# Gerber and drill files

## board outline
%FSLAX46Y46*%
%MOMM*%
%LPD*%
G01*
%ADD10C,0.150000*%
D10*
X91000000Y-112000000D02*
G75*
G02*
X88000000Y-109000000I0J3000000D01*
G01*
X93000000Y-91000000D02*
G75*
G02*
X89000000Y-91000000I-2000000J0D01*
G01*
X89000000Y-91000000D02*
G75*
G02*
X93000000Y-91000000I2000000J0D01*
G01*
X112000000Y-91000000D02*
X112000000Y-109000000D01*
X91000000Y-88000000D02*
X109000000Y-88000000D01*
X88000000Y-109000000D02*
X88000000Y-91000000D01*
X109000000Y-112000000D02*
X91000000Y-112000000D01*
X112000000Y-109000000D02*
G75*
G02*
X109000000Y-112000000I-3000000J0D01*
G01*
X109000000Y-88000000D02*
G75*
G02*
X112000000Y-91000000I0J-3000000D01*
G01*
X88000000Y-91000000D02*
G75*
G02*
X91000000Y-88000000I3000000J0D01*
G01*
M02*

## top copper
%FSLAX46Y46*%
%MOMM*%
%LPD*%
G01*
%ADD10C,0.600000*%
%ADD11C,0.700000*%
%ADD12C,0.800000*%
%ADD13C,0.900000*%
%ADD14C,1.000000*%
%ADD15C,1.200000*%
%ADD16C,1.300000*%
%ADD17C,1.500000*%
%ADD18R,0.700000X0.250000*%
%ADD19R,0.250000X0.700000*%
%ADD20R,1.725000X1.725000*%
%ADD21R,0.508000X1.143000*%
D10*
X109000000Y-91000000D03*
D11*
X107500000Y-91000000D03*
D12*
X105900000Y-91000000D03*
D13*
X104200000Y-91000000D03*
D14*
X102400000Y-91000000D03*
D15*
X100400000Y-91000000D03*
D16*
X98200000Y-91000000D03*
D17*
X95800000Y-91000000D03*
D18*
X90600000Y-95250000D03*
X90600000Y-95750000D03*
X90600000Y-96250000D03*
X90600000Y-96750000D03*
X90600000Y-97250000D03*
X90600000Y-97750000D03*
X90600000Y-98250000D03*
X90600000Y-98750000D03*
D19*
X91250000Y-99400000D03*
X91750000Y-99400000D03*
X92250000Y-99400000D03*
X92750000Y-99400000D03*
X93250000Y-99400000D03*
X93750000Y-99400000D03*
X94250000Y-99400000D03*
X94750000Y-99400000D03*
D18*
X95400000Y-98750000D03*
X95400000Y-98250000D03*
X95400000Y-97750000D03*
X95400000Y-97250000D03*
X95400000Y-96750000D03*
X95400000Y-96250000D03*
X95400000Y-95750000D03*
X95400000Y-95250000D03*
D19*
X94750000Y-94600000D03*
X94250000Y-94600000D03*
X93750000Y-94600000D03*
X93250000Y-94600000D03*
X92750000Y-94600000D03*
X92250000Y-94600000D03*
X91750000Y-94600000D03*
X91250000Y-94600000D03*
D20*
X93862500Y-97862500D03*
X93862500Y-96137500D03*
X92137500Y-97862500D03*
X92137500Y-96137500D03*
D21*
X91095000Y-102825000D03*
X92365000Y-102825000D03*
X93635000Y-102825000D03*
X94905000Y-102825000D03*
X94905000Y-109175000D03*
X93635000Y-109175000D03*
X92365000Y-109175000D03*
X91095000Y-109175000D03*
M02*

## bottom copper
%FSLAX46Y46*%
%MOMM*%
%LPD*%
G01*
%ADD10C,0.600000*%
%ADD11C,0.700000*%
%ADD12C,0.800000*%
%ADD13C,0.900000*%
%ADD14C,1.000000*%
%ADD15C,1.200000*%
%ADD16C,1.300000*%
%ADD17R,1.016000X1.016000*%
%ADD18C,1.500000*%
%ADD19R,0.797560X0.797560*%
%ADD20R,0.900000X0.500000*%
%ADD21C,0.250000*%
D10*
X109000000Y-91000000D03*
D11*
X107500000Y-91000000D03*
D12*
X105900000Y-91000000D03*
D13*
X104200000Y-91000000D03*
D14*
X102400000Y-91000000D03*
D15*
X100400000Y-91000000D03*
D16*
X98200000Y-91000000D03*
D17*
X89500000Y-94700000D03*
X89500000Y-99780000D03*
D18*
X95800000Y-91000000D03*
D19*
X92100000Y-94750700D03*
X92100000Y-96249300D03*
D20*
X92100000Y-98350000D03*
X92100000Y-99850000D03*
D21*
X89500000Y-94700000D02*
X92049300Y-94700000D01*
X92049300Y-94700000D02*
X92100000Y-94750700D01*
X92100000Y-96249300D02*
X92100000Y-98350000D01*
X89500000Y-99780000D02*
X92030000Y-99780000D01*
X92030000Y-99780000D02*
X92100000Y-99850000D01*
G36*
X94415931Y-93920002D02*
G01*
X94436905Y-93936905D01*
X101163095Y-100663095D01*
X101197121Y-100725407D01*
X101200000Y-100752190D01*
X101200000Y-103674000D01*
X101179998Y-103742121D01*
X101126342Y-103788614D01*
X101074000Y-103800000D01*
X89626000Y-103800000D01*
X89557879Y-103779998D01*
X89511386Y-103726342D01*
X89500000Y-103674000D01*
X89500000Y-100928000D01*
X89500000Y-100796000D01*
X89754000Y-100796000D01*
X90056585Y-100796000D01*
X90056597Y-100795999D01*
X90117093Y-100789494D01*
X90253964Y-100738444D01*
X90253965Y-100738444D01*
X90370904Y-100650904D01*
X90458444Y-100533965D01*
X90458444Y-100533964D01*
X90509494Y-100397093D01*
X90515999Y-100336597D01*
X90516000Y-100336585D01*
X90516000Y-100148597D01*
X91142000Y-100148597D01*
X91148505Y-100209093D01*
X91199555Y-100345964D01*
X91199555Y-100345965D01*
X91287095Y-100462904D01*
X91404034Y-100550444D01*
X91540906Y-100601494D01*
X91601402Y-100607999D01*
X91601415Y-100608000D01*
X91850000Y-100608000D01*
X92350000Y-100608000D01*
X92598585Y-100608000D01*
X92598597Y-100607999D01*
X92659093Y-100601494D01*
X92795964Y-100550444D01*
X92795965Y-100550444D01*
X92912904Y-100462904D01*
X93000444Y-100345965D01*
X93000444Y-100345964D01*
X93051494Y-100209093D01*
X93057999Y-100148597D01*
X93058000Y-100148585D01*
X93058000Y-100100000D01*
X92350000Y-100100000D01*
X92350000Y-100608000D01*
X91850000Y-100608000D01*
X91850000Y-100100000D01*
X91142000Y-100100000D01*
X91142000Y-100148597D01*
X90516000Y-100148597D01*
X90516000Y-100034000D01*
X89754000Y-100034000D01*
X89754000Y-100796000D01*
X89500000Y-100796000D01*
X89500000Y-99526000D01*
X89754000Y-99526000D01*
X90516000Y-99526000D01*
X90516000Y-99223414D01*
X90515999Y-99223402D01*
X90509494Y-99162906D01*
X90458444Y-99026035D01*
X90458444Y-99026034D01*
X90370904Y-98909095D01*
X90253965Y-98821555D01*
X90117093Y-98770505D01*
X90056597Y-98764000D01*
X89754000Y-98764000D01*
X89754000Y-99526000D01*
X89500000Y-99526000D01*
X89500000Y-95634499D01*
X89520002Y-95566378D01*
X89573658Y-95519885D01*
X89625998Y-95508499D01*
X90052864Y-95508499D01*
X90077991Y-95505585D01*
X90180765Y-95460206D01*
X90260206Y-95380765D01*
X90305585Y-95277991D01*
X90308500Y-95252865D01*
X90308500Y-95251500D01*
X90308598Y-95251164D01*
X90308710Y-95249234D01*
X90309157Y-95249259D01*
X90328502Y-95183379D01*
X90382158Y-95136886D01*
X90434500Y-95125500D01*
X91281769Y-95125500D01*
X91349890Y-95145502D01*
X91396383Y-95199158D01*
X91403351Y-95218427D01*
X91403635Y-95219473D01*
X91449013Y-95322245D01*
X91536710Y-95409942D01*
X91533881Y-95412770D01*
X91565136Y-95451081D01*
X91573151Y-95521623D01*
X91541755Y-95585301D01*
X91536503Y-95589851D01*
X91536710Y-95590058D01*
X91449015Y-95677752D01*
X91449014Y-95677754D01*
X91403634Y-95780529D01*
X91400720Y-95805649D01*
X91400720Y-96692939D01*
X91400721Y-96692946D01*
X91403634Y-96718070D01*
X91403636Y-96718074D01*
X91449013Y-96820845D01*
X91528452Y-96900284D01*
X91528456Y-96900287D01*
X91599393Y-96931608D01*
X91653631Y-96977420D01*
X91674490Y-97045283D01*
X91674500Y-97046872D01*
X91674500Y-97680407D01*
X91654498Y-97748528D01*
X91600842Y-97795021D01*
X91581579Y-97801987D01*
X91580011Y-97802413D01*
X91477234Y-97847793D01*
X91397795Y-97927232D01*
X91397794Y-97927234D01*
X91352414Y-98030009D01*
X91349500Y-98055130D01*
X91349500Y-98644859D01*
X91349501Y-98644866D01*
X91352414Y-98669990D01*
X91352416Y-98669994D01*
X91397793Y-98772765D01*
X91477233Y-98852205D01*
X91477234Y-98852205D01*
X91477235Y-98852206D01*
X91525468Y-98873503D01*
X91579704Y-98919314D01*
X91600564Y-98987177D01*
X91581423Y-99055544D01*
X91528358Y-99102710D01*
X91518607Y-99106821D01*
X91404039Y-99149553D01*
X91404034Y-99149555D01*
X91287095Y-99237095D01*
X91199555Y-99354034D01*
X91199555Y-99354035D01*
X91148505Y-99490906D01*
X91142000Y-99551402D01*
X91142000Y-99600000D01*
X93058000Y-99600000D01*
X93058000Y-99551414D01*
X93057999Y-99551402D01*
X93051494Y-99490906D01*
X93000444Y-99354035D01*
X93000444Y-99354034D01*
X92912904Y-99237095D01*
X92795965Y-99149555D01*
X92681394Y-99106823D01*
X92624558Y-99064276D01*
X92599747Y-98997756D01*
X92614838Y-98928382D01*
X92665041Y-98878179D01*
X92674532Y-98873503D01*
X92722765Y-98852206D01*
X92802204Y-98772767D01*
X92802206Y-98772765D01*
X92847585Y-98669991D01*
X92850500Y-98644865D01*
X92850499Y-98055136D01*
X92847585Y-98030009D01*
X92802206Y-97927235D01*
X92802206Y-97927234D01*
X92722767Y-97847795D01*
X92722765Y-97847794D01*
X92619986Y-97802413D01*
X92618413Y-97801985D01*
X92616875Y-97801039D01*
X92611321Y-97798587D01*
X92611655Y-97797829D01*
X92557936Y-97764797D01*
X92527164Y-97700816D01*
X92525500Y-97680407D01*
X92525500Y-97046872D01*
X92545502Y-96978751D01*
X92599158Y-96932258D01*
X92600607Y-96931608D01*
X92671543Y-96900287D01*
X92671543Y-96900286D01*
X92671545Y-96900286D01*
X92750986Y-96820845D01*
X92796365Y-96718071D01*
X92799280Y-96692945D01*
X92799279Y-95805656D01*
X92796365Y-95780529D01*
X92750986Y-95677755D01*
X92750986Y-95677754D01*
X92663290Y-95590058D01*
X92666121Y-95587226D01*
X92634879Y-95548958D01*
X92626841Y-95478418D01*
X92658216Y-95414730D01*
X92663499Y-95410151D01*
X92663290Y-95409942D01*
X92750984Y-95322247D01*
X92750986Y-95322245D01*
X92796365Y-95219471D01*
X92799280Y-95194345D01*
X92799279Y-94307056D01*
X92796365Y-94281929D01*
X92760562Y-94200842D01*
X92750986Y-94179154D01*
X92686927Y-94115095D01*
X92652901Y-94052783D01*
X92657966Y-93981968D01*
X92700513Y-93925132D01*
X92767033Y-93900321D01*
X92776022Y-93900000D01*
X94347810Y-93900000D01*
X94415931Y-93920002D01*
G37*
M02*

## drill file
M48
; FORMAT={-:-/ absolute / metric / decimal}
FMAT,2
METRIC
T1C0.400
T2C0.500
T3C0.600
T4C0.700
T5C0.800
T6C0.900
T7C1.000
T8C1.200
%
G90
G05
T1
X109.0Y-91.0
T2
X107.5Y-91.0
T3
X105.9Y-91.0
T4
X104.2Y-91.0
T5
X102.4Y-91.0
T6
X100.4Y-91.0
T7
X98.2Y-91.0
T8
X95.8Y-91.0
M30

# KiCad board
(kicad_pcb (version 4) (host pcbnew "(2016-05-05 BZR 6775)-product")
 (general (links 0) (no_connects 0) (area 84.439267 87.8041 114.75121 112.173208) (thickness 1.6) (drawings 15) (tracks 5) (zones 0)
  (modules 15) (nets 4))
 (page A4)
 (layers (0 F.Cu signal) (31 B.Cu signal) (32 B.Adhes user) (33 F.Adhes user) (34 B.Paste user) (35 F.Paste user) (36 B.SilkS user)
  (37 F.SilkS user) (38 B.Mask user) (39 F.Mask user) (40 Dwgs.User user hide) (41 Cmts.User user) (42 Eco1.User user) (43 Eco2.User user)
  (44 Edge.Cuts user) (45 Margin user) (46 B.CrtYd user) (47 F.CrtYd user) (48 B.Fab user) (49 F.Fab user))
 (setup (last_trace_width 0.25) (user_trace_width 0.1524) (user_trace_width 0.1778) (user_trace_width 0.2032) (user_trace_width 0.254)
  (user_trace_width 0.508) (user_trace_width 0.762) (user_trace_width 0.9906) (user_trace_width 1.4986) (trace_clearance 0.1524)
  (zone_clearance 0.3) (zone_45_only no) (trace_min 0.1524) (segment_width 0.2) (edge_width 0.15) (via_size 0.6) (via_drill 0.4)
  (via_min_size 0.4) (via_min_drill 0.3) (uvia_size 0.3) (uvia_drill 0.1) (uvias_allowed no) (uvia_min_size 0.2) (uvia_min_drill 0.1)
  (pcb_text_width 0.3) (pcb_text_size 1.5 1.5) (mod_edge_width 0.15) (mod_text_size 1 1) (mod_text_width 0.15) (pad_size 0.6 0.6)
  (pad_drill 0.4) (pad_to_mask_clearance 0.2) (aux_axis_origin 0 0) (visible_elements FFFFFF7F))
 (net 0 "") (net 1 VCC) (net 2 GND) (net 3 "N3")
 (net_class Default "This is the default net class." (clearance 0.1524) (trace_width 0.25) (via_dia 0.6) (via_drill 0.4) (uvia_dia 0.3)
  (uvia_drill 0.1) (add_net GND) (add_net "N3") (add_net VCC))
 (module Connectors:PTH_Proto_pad (layer F.Cu) (at 109 91)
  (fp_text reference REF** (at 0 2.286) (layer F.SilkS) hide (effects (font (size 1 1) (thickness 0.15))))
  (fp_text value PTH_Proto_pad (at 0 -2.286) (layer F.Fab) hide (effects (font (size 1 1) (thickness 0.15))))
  (pad 1 thru_hole circle (at 0 0) (size 0.6 0.6) (drill 0.4) (layers *.Cu *.Mask F.SilkS)))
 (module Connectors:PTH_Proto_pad (layer F.Cu) (at 107.5 91)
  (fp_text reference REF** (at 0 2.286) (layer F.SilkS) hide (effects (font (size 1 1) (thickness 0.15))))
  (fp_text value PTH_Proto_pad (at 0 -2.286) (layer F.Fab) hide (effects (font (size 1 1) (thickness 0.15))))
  (pad 1 thru_hole circle (at 0 0) (size 0.7 0.7) (drill 0.5) (layers *.Cu *.Mask F.SilkS)))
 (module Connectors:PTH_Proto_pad (layer F.Cu) (at 105.9 91)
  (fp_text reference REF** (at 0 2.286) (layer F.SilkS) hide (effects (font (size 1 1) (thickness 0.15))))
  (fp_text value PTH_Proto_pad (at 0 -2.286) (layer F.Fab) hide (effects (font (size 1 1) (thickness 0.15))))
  (pad 1 thru_hole circle (at 0 0) (size 0.8 0.8) (drill 0.6) (layers *.Cu *.Mask F.SilkS)))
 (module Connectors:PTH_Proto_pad (layer F.Cu) (at 104.2 91)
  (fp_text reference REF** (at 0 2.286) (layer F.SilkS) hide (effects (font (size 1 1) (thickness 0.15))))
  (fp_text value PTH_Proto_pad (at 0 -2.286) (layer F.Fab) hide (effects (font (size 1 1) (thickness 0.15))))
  (pad 1 thru_hole circle (at 0 0) (size 0.9 0.9) (drill 0.7) (layers *.Cu *.Mask F.SilkS)))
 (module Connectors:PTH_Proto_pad (layer F.Cu) (at 102.4 91)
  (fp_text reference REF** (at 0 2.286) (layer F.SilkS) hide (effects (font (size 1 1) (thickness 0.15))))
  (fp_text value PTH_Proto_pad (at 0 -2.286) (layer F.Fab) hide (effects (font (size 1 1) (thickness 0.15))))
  (pad 1 thru_hole circle (at 0 0) (size 1 1) (drill 0.8) (layers *.Cu *.Mask F.SilkS)))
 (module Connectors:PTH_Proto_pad (layer F.Cu) (at 100.4 91)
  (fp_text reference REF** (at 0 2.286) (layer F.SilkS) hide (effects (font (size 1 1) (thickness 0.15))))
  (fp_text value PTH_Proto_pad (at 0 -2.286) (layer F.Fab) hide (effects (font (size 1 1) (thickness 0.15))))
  (pad 1 thru_hole circle (at 0 0) (size 1.2 1.2) (drill 0.9) (layers *.Cu *.Mask F.SilkS)))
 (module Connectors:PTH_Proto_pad (layer F.Cu) (at 98.2 91)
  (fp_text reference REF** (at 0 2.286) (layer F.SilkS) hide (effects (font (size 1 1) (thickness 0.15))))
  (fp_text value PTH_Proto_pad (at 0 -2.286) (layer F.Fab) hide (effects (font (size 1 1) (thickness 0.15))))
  (pad 1 thru_hole circle (at 0 0) (size 1.3 1.3) (drill 1) (layers *.Cu *.Mask F.SilkS)))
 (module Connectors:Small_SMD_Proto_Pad (layer B.Cu) (at 89.5 94.7)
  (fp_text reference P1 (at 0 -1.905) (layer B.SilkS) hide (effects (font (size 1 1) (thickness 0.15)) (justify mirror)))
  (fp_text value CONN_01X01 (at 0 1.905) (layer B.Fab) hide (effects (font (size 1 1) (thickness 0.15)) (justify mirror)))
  (pad 1 smd rect (at 0 0) (size 1.016 1.016) (layers B.Cu B.Paste B.Mask) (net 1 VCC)))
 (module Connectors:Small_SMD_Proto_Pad (layer B.Cu) (at 89.5 99.78)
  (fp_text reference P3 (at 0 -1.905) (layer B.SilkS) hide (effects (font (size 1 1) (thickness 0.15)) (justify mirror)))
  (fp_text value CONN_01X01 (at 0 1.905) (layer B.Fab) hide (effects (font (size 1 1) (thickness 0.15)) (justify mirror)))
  (pad 1 smd rect (at 0 0) (size 1.016 1.016) (layers B.Cu B.Paste B.Mask) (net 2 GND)))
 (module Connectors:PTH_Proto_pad (layer F.Cu) (at 95.8 91)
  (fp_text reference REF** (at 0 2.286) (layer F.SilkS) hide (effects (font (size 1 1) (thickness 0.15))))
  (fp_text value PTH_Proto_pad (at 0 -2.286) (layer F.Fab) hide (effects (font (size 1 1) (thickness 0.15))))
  (pad 1 thru_hole circle (at 0 0) (size 1.5 1.5) (drill 1.2) (layers *.Cu *.Mask F.SilkS)))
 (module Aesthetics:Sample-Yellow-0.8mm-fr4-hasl (layer B.Cu) (at 100 102.6 180)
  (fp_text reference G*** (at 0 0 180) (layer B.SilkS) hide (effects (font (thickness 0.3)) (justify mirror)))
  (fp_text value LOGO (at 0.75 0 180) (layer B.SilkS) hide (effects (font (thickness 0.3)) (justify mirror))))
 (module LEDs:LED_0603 (layer B.Cu) (at 92.1 95.5 90)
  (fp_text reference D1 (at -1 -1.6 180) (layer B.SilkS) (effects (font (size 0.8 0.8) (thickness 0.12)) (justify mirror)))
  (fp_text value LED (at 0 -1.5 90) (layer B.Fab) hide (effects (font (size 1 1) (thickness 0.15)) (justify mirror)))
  (pad 2 smd rect (at 0.7493 0 270) (size 0.79756 0.79756) (layers B.Cu B.Paste B.Mask) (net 1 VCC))
  (pad 1 smd rect (at -0.7493 0 270) (size 0.79756 0.79756) (layers B.Cu B.Paste B.Mask) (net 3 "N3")))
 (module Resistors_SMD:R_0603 (layer B.Cu) (at 92.1 99.1 270)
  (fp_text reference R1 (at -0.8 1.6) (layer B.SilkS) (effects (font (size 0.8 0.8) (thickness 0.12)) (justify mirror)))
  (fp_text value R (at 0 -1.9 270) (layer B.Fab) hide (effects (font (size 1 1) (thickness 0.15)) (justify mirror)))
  (pad 1 smd rect (at -0.75 0 270) (size 0.5 0.9) (layers B.Cu B.Paste B.Mask) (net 3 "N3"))
  (pad 2 smd rect (at 0.75 0 270) (size 0.5 0.9) (layers B.Cu B.Paste B.Mask) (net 2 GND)))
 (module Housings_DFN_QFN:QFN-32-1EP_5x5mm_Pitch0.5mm (layer F.Cu) (at 93 97)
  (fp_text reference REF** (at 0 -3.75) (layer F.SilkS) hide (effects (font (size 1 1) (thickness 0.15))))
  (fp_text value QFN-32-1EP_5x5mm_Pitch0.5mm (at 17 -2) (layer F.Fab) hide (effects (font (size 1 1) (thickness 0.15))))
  (pad 1 smd rect (at -2.4 -1.75) (size 0.7 0.25) (layers F.Cu F.Paste F.Mask))
  (pad 2 smd rect (at -2.4 -1.25) (size 0.7 0.25) (layers F.Cu F.Paste F.Mask))
  (pad 3 smd rect (at -2.4 -0.75) (size 0.7 0.25) (layers F.Cu F.Paste F.Mask))
  (pad 4 smd rect (at -2.4 -0.25) (size 0.7 0.25) (layers F.Cu F.Paste F.Mask))
  (pad 5 smd rect (at -2.4 0.25) (size 0.7 0.25) (layers F.Cu F.Paste F.Mask))
  (pad 6 smd rect (at -2.4 0.75) (size 0.7 0.25) (layers F.Cu F.Paste F.Mask))
  (pad 7 smd rect (at -2.4 1.25) (size 0.7 0.25) (layers F.Cu F.Paste F.Mask))
  (pad 8 smd rect (at -2.4 1.75) (size 0.7 0.25) (layers F.Cu F.Paste F.Mask))
  (pad 9 smd rect (at -1.75 2.4 90) (size 0.7 0.25) (layers F.Cu F.Paste F.Mask))
  (pad 10 smd rect (at -1.25 2.4 90) (size 0.7 0.25) (layers F.Cu F.Paste F.Mask))
  (pad 11 smd rect (at -0.75 2.4 90) (size 0.7 0.25) (layers F.Cu F.Paste F.Mask))
  (pad 12 smd rect (at -0.25 2.4 90) (size 0.7 0.25) (layers F.Cu F.Paste F.Mask))
  (pad 13 smd rect (at 0.25 2.4 90) (size 0.7 0.25) (layers F.Cu F.Paste F.Mask))
  (pad 14 smd rect (at 0.75 2.4 90) (size 0.7 0.25) (layers F.Cu F.Paste F.Mask))
  (pad 15 smd rect (at 1.25 2.4 90) (size 0.7 0.25) (layers F.Cu F.Paste F.Mask))
  (pad 16 smd rect (at 1.75 2.4 90) (size 0.7 0.25) (layers F.Cu F.Paste F.Mask))
  (pad 17 smd rect (at 2.4 1.75) (size 0.7 0.25) (layers F.Cu F.Paste F.Mask))
  (pad 18 smd rect (at 2.4 1.25) (size 0.7 0.25) (layers F.Cu F.Paste F.Mask))
  (pad 19 smd rect (at 2.4 0.75) (size 0.7 0.25) (layers F.Cu F.Paste F.Mask))
  (pad 20 smd rect (at 2.4 0.25) (size 0.7 0.25) (layers F.Cu F.Paste F.Mask))
  (pad 21 smd rect (at 2.4 -0.25) (size 0.7 0.25) (layers F.Cu F.Paste F.Mask))
  (pad 22 smd rect (at 2.4 -0.75) (size 0.7 0.25) (layers F.Cu F.Paste F.Mask))
  (pad 23 smd rect (at 2.4 -1.25) (size 0.7 0.25) (layers F.Cu F.Paste F.Mask))
  (pad 24 smd rect (at 2.4 -1.75) (size 0.7 0.25) (layers F.Cu F.Paste F.Mask))
  (pad 25 smd rect (at 1.75 -2.4 90) (size 0.7 0.25) (layers F.Cu F.Paste F.Mask))
  (pad 26 smd rect (at 1.25 -2.4 90) (size 0.7 0.25) (layers F.Cu F.Paste F.Mask))
  (pad 27 smd rect (at 0.75 -2.4 90) (size 0.7 0.25) (layers F.Cu F.Paste F.Mask))
  (pad 28 smd rect (at 0.25 -2.4 90) (size 0.7 0.25) (layers F.Cu F.Paste F.Mask))
  (pad 29 smd rect (at -0.25 -2.4 90) (size 0.7 0.25) (layers F.Cu F.Paste F.Mask))
  (pad 30 smd rect (at -0.75 -2.4 90) (size 0.7 0.25) (layers F.Cu F.Paste F.Mask))
  (pad 31 smd rect (at -1.25 -2.4 90) (size 0.7 0.25) (layers F.Cu F.Paste F.Mask))
  (pad 32 smd rect (at -1.75 -2.4 90) (size 0.7 0.25) (layers F.Cu F.Paste F.Mask))
  (pad 33 smd rect (at 0.8625 0.8625) (size 1.725 1.725) (layers F.Cu F.Paste F.Mask) (solder_paste_margin_ratio -0.2))
  (pad 33 smd rect (at 0.8625 -0.8625) (size 1.725 1.725) (layers F.Cu F.Paste F.Mask) (solder_paste_margin_ratio -0.2))
  (pad 33 smd rect (at -0.8625 0.8625) (size 1.725 1.725) (layers F.Cu F.Paste F.Mask) (solder_paste_margin_ratio -0.2))
  (pad 33 smd rect (at -0.8625 -0.8625) (size 1.725 1.725) (layers F.Cu F.Paste F.Mask) (solder_paste_margin_ratio -0.2)))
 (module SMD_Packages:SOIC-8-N (layer F.Cu) (at 93 106)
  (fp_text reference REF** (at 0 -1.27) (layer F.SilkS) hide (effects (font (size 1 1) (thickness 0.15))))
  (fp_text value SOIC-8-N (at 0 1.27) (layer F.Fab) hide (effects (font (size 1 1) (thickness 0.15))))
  (pad 8 smd rect (at -1.905 -3.175) (size 0.508 1.143) (layers F.Cu F.Paste F.Mask))
  (pad 7 smd rect (at -0.635 -3.175) (size 0.508 1.143) (layers F.Cu F.Paste F.Mask))
  (pad 6 smd rect (at 0.635 -3.175) (size 0.508 1.143) (layers F.Cu F.Paste F.Mask))
  (pad 5 smd rect (at 1.905 -3.175) (size 0.508 1.143) (layers F.Cu F.Paste F.Mask))
  (pad 4 smd rect (at 1.905 3.175) (size 0.508 1.143) (layers F.Cu F.Paste F.Mask))
  (pad 3 smd rect (at 0.635 3.175) (size 0.508 1.143) (layers F.Cu F.Paste F.Mask))
  (pad 2 smd rect (at -0.635 3.175) (size 0.508 1.143) (layers F.Cu F.Paste F.Mask))
  (pad 1 smd rect (at -1.905 3.175) (size 0.508 1.143) (layers F.Cu F.Paste F.Mask)))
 (gr_arc (start 91 109) (end 91 112) (angle 90) (layer Edge.Cuts) (width 0.15))
 (gr_circle (center 91 91) (end 93 91) (layer Edge.Cuts) (width 0.15))
 (gr_line (start 112 91) (end 112 109) (layer Edge.Cuts) (width 0.15))
 (gr_line (start 91 88) (end 109 88) (layer Edge.Cuts) (width 0.15))
 (gr_line (start 88 109) (end 88 91) (layer Edge.Cuts) (width 0.15))
 (gr_line (start 109 112) (end 91 112) (layer Edge.Cuts) (width 0.15))
 (gr_arc (start 109 109) (end 112 109) (angle 90) (layer Edge.Cuts) (width 0.15))
 (gr_arc (start 109 91) (end 109 88) (angle 90) (layer Edge.Cuts) (width 0.15))
 (gr_arc (start 91 91) (end 88 91) (angle 90) (layer Edge.Cuts) (width 0.15))
 (segment (start 89.5 94.7) (end 92.0493 94.7) (width 0.25) (layer B.Cu) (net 1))
 (segment (start 92.0493 94.7) (end 92.1 94.7507) (width 0.25) (layer B.Cu) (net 1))
 (segment (start 92.1 96.2493) (end 92.1 98.35) (width 0.25) (layer B.Cu) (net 3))
 (segment (start 89.5 99.78) (end 92.03 99.78) (width 0.25) (layer B.Cu) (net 2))
 (segment (start 92.03 99.78) (end 92.1 99.85) (width 0.25) (layer B.Cu) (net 2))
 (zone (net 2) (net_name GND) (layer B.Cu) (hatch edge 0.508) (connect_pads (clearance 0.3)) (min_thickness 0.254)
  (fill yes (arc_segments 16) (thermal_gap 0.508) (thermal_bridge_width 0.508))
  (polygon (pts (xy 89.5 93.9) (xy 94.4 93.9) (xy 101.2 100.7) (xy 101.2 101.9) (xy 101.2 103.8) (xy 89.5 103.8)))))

